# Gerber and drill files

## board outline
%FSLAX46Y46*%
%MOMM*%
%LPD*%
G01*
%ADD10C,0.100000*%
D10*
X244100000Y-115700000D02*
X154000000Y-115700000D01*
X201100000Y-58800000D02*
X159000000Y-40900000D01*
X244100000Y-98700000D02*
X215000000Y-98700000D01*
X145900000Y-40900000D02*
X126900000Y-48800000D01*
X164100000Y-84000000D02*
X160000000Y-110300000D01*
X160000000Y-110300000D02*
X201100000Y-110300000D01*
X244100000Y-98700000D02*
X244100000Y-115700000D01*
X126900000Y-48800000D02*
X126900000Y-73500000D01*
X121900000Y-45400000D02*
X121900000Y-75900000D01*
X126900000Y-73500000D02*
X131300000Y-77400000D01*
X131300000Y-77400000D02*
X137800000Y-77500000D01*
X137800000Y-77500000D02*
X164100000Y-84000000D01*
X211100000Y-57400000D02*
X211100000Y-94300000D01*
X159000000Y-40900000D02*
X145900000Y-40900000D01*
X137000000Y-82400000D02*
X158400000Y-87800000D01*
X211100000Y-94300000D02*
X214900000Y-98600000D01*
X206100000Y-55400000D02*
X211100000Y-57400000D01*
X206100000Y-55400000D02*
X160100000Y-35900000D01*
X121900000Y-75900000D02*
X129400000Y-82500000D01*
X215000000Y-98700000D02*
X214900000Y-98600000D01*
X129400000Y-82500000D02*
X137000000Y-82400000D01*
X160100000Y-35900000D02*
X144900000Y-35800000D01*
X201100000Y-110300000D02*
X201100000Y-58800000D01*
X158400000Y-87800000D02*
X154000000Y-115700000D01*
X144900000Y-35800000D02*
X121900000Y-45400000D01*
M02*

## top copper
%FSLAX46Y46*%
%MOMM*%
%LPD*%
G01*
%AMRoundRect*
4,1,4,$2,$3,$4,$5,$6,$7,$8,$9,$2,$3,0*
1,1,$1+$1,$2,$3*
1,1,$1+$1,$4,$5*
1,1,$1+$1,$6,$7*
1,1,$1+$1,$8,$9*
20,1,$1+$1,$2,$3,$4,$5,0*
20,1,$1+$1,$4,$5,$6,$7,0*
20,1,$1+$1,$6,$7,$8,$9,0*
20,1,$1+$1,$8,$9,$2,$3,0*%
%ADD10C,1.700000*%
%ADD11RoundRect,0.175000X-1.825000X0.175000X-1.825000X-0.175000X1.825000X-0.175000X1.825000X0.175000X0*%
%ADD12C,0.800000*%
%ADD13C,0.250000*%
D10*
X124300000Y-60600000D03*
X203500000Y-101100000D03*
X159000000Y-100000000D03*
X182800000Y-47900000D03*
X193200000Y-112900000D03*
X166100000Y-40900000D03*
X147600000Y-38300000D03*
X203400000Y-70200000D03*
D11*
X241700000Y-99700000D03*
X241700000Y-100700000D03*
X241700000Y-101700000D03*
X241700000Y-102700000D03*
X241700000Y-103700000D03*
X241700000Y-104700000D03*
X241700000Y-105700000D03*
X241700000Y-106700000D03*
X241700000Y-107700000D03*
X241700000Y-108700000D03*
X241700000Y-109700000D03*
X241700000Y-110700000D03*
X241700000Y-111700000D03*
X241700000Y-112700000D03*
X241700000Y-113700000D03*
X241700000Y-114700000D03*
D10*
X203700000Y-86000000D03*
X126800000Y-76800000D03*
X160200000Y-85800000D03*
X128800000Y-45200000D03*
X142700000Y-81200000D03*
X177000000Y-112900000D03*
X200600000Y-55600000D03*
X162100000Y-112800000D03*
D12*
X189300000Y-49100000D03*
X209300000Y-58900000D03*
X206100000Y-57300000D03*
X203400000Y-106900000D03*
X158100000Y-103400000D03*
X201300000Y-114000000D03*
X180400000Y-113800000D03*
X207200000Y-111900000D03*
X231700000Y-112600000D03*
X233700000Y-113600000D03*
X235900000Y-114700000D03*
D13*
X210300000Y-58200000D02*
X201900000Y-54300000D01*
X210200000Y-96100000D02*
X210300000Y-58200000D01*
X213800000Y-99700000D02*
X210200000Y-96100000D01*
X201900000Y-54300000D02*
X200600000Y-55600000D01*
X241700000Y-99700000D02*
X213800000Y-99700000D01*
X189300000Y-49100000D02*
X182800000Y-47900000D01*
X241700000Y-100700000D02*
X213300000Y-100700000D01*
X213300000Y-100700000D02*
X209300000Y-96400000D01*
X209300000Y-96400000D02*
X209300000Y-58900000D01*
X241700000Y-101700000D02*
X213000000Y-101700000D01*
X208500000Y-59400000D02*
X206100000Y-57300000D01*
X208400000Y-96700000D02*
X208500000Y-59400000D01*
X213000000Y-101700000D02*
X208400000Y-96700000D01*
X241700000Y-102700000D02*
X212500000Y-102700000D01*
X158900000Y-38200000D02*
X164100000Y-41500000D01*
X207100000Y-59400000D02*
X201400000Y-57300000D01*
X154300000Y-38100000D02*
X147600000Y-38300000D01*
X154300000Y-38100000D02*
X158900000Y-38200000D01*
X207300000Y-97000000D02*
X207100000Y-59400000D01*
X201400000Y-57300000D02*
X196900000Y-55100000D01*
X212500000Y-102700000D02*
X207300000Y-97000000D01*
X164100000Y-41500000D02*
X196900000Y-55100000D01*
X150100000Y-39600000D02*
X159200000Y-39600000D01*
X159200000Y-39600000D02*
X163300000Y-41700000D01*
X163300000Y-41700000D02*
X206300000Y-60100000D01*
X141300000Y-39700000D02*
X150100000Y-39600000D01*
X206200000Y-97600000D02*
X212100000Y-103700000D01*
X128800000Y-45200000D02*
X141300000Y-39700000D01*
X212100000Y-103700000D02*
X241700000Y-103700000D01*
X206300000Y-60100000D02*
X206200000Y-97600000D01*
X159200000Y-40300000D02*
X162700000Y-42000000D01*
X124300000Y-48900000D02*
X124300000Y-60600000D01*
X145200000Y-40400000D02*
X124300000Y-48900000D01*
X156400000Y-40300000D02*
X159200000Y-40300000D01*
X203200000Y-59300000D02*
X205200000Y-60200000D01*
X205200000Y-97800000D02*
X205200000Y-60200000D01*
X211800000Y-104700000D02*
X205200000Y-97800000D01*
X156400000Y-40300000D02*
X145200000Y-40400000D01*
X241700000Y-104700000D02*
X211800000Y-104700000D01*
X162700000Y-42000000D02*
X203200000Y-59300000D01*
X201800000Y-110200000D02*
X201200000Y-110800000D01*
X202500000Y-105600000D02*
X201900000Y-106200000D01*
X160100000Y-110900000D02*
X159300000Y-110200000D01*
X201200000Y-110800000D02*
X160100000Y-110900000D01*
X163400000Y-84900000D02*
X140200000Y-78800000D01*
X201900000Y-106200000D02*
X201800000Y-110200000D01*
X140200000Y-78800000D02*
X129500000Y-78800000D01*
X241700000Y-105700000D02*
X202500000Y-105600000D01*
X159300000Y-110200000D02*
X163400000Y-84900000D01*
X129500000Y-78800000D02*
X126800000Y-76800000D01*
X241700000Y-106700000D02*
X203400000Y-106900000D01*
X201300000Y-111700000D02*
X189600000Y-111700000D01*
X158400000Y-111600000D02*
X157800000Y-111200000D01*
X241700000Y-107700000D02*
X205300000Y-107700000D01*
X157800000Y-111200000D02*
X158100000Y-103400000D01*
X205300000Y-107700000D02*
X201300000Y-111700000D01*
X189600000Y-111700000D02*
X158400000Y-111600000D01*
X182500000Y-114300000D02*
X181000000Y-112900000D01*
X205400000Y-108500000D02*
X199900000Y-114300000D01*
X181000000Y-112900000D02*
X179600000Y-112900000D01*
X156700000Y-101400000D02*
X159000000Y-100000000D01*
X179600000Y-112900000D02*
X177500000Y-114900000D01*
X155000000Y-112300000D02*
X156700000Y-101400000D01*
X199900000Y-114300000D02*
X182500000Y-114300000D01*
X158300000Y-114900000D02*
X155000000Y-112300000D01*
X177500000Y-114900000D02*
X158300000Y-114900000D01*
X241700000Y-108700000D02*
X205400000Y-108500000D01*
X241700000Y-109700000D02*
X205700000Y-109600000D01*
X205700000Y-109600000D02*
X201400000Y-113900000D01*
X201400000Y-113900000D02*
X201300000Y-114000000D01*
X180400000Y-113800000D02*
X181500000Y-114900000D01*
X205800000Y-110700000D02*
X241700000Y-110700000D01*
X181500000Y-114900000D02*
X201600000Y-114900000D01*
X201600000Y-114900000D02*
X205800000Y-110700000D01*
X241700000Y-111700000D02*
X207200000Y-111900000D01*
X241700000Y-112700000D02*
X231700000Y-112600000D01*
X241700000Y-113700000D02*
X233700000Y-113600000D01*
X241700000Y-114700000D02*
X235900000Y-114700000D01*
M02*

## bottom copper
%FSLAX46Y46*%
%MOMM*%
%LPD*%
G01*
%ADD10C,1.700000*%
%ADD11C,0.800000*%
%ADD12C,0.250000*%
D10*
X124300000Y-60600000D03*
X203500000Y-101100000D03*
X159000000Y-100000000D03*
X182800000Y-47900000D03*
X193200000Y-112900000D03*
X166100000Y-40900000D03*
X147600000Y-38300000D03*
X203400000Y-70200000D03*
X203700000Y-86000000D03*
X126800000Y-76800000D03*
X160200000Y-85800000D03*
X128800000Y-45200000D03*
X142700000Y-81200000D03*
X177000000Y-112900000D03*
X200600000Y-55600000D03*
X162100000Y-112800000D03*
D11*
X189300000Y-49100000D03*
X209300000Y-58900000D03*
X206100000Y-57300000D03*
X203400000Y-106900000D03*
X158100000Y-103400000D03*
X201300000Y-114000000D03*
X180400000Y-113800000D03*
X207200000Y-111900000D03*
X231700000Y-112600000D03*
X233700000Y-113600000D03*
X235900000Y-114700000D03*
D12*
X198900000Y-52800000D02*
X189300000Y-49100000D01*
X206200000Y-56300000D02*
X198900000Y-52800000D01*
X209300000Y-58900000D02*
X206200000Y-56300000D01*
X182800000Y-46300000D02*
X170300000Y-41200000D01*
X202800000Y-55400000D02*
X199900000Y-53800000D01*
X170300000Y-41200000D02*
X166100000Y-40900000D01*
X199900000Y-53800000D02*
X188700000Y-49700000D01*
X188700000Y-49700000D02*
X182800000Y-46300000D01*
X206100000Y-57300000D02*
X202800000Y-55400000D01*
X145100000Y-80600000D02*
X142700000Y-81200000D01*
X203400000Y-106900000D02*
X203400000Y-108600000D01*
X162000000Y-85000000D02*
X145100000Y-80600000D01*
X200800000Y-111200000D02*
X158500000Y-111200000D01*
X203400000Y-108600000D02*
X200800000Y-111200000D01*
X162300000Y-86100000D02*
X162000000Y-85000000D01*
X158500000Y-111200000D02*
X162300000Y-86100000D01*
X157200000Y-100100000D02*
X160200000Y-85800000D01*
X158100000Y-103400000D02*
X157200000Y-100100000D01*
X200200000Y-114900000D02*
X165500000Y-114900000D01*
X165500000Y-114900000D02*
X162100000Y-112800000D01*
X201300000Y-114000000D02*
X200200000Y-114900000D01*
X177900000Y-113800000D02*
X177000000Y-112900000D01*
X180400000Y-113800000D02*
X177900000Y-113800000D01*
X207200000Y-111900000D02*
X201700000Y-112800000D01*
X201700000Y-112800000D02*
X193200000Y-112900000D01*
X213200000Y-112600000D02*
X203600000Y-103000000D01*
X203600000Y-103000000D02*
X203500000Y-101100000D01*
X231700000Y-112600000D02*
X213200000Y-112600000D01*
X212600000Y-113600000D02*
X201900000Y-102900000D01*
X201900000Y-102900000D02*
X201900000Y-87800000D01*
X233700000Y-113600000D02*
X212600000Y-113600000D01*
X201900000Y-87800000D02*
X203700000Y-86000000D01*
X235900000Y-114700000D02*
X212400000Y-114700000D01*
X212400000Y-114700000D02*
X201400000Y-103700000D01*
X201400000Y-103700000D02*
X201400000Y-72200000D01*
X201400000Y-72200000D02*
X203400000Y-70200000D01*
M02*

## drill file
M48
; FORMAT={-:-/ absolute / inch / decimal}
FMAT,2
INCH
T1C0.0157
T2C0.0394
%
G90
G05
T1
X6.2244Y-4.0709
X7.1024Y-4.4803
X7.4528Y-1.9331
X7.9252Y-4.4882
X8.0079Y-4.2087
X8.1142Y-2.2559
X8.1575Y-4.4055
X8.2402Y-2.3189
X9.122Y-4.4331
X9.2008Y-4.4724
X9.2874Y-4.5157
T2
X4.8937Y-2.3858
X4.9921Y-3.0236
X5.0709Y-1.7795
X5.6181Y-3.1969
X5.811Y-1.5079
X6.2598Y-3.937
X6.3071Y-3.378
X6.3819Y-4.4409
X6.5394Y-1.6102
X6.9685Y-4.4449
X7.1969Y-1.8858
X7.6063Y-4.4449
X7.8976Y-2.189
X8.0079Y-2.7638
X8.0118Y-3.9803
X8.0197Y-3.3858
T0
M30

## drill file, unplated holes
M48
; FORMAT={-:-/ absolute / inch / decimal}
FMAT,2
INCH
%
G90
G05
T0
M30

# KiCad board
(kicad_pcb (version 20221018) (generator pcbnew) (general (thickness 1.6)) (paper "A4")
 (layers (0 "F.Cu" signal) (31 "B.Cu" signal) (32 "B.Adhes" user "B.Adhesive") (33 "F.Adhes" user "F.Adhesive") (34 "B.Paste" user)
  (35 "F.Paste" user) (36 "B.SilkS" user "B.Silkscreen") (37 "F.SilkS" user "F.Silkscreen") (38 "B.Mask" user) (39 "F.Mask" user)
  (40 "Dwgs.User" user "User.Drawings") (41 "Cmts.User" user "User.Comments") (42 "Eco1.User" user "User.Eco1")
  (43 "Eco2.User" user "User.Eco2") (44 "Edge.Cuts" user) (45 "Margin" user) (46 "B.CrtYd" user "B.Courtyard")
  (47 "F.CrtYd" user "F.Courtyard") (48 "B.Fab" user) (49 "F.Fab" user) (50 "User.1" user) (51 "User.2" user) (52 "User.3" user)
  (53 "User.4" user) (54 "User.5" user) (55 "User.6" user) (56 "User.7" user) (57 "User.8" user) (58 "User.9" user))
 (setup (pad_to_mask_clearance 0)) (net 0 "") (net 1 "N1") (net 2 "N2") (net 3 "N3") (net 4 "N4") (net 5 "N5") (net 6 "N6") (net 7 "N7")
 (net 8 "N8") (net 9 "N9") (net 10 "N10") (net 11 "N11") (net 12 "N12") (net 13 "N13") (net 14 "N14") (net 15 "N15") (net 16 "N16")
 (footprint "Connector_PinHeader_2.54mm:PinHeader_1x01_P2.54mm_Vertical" (layer "F.Cu") (at 124.3 60.6)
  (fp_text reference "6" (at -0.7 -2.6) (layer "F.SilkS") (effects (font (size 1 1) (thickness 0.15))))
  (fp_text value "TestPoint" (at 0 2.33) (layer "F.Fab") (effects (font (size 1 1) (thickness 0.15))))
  (pad "1" thru_hole circle (at 0 0) (size 1.7 1.7) (drill 1) (layers "*.Cu" "*.Mask") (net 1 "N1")))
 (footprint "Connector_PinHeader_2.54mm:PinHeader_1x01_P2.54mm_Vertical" (layer "F.Cu") (at 203.5 101.1)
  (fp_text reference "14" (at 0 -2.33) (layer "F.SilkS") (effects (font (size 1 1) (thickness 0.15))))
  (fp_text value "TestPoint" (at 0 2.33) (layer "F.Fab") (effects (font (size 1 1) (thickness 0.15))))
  (pad "1" thru_hole circle (at 0 0) (size 1.7 1.7) (drill 1) (layers "*.Cu" "*.Mask") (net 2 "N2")))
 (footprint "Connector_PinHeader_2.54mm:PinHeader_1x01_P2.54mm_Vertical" (layer "F.Cu") (at 159 100)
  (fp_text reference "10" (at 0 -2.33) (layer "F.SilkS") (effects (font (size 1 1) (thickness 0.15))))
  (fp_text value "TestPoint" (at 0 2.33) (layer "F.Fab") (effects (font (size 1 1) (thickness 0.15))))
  (pad "1" thru_hole circle (at 0 0) (size 1.7 1.7) (drill 1) (layers "*.Cu" "*.Mask") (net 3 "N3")))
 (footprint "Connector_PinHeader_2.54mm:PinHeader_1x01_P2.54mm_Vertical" (layer "F.Cu") (at 182.8 47.9)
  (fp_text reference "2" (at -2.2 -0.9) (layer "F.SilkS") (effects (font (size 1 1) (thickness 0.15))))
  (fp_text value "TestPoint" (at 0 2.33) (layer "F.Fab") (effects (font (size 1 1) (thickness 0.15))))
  (pad "1" thru_hole circle (at 0 0) (size 1.7 1.7) (drill 1) (layers "*.Cu" "*.Mask") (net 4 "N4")))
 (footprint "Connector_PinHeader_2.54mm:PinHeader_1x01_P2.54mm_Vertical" (layer "F.Cu") (at 193.2 112.9)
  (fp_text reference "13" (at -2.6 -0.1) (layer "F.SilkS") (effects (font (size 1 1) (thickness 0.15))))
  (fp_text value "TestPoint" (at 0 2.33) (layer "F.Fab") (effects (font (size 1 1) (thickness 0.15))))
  (pad "1" thru_hole circle (at 0 0) (size 1.7 1.7) (drill 1) (layers "*.Cu" "*.Mask") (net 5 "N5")))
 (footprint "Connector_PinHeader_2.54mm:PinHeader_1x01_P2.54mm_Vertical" (layer "F.Cu") (at 166.1 40.9)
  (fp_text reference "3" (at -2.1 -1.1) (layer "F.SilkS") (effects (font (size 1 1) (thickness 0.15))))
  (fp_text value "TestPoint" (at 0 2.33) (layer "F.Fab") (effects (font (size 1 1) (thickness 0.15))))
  (pad "1" thru_hole circle (at 0 0) (size 1.7 1.7) (drill 1) (layers "*.Cu" "*.Mask") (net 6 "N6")))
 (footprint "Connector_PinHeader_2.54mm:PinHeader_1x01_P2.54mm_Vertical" (layer "F.Cu") (at 147.6 38.3)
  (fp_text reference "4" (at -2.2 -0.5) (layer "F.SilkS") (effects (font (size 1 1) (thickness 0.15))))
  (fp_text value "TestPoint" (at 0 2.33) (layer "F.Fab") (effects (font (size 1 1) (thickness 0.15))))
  (pad "1" thru_hole circle (at 0 0) (size 1.7 1.7) (drill 1) (layers "*.Cu" "*.Mask") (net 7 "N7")))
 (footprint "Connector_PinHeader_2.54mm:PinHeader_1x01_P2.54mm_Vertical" (layer "F.Cu") (at 203.4 70.2)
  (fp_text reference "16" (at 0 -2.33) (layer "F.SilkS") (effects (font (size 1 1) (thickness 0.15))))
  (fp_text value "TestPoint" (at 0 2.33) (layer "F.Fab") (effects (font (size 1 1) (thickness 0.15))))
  (pad "1" thru_hole circle (at 0 0) (size 1.7 1.7) (drill 1) (layers "*.Cu" "*.Mask") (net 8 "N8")))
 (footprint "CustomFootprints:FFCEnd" (layer "F.Cu") (at 238.7 107.2 -90)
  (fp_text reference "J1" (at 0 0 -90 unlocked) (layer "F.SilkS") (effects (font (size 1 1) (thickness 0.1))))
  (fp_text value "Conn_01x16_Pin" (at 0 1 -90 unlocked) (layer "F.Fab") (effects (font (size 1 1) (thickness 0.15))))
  (pad "1" smd roundrect (at -7.5 -3 270) (size 0.7 4) (layers "F.Cu" "F.Paste" "F.Mask") (roundrect_rratio 0.25) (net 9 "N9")
   (thermal_bridge_angle 45))
  (pad "2" smd roundrect (at -6.5 -3 270) (size 0.7 4) (layers "F.Cu" "F.Paste" "F.Mask") (roundrect_rratio 0.25) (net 4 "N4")
   (thermal_bridge_angle 45))
  (pad "3" smd roundrect (at -5.5 -3 270) (size 0.7 4) (layers "F.Cu" "F.Paste" "F.Mask") (roundrect_rratio 0.25) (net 6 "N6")
   (thermal_bridge_angle 45))
  (pad "4" smd roundrect (at -4.5 -3 270) (size 0.7 4) (layers "F.Cu" "F.Paste" "F.Mask") (roundrect_rratio 0.25) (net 7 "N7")
   (thermal_bridge_angle 45))
  (pad "5" smd roundrect (at -3.5 -3 270) (size 0.7 4) (layers "F.Cu" "F.Paste" "F.Mask") (roundrect_rratio 0.25) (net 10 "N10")
   (thermal_bridge_angle 45))
  (pad "6" smd roundrect (at -2.5 -3 270) (size 0.7 4) (layers "F.Cu" "F.Paste" "F.Mask") (roundrect_rratio 0.25) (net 1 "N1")
   (thermal_bridge_angle 45))
  (pad "7" smd roundrect (at -1.5 -3 270) (size 0.7 4) (layers "F.Cu" "F.Paste" "F.Mask") (roundrect_rratio 0.25) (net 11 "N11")
   (thermal_bridge_angle 45))
  (pad "8" smd roundrect (at -0.5 -3 270) (size 0.7 4) (layers "F.Cu" "F.Paste" "F.Mask") (roundrect_rratio 0.25) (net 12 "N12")
   (thermal_bridge_angle 45))
  (pad "9" smd roundrect (at 0.5 -3 270) (size 0.7 4) (layers "F.Cu" "F.Paste" "F.Mask") (roundrect_rratio 0.25) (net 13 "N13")
   (thermal_bridge_angle 45))
  (pad "10" smd roundrect (at 1.5 -3 270) (size 0.7 4) (layers "F.Cu" "F.Paste" "F.Mask") (roundrect_rratio 0.25) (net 3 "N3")
   (thermal_bridge_angle 45))
  (pad "11" smd roundrect (at 2.5 -3 270) (size 0.7 4) (layers "F.Cu" "F.Paste" "F.Mask") (roundrect_rratio 0.25) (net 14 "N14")
   (thermal_bridge_angle 45))
  (pad "12" smd roundrect (at 3.5 -3 270) (size 0.7 4) (layers "F.Cu" "F.Paste" "F.Mask") (roundrect_rratio 0.25) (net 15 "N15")
   (thermal_bridge_angle 45))
  (pad "13" smd roundrect (at 4.5 -3 270) (size 0.7 4) (layers "F.Cu" "F.Paste" "F.Mask") (roundrect_rratio 0.25) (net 5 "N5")
   (thermal_bridge_angle 45))
  (pad "14" smd roundrect (at 5.5 -3 270) (size 0.7 4) (layers "F.Cu" "F.Paste" "F.Mask") (roundrect_rratio 0.25) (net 2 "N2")
   (thermal_bridge_angle 45))
  (pad "15" smd roundrect (at 6.5 -3 270) (size 0.7 4) (layers "F.Cu" "F.Paste" "F.Mask") (roundrect_rratio 0.25) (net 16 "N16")
   (thermal_bridge_angle 45))
  (pad "16" smd roundrect (at 7.5 -3 270) (size 0.7 4) (layers "F.Cu" "F.Paste" "F.Mask") (roundrect_rratio 0.25) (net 8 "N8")
   (thermal_bridge_angle 45)))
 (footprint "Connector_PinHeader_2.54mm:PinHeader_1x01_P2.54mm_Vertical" (layer "F.Cu") (at 203.7 86)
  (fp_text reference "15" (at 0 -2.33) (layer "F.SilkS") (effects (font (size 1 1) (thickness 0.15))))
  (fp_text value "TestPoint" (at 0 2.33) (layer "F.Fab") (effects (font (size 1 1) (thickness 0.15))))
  (pad "1" thru_hole circle (at 0 0) (size 1.7 1.7) (drill 1) (layers "*.Cu" "*.Mask") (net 16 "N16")))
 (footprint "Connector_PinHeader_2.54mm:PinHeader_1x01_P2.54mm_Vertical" (layer "F.Cu") (at 126.8 76.8)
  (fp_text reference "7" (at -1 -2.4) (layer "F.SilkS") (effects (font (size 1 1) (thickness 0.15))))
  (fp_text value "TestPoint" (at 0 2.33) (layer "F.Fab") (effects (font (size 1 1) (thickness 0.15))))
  (pad "1" thru_hole circle (at 0 0) (size 1.7 1.7) (drill 1) (layers "*.Cu" "*.Mask") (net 11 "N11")))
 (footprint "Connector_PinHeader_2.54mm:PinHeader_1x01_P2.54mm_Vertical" (layer "F.Cu") (at 160.2 85.8)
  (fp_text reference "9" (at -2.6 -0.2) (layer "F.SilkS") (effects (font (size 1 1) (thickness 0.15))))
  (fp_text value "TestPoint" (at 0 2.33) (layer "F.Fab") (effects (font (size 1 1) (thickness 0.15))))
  (pad "1" thru_hole circle (at 0 0) (size 1.7 1.7) (drill 1) (layers "*.Cu" "*.Mask") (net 13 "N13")))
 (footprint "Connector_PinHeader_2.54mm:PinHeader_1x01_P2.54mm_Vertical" (layer "F.Cu") (at 128.8 45.2)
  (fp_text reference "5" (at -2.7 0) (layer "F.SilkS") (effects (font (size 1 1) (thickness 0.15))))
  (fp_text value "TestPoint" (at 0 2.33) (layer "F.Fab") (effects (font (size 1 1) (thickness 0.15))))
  (pad "1" thru_hole circle (at 0 0) (size 1.7 1.7) (drill 1) (layers "*.Cu" "*.Mask") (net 10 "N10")))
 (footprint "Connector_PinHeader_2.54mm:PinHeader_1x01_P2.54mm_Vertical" (layer "F.Cu") (at 142.7 81.2)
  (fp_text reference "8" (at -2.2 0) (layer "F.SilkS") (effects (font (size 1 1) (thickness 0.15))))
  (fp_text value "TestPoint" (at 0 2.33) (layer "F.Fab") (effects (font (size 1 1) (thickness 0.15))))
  (pad "1" thru_hole circle (at 0 0) (size 1.7 1.7) (drill 1) (layers "*.Cu" "*.Mask") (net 12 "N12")))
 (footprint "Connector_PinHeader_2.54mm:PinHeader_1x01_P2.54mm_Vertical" (layer "F.Cu") (at 177 112.9)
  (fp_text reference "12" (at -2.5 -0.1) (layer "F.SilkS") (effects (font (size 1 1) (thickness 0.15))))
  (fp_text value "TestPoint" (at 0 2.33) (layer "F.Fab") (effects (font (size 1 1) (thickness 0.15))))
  (pad "1" thru_hole circle (at 0 0) (size 1.7 1.7) (drill 1) (layers "*.Cu" "*.Mask") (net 15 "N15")))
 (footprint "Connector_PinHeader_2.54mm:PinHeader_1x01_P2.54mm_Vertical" (layer "F.Cu") (at 200.6 55.6)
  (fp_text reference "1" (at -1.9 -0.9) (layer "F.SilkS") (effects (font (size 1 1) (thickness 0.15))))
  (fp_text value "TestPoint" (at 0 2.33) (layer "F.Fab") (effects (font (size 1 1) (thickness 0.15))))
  (pad "1" thru_hole circle (at 0 0) (size 1.7 1.7) (drill 1) (layers "*.Cu" "*.Mask") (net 9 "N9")))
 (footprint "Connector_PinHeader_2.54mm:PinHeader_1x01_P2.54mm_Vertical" (layer "F.Cu") (at 162.1 112.8)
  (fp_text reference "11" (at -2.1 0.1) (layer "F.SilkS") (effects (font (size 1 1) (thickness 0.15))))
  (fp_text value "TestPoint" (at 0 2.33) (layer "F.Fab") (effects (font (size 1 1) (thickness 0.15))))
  (pad "1" thru_hole circle (at 0 0) (size 1.7 1.7) (drill 1) (layers "*.Cu" "*.Mask") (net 14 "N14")))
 (gr_line (start 201.1 58.8) (end 159 40.9) (stroke (width 0.1) (type default)) (layer "Edge.Cuts"))
 (gr_line (start 244.1 98.7) (end 215 98.7) (stroke (width 0.1) (type default)) (layer "Edge.Cuts"))
 (gr_line (start 244.1 115.7) (end 154 115.7) (stroke (width 0.1) (type default)) (layer "Edge.Cuts"))
 (gr_line (start 145.9 40.9) (end 126.9 48.8) (stroke (width 0.1) (type default)) (layer "Edge.Cuts"))
 (gr_line (start 164.1 84) (end 160 110.3) (stroke (width 0.1) (type default)) (layer "Edge.Cuts"))
 (gr_line (start 160 110.3) (end 201.1 110.3) (stroke (width 0.1) (type default)) (layer "Edge.Cuts"))
 (gr_line (start 244.1 98.7) (end 244.1 115.7) (stroke (width 0.1) (type default)) (layer "Edge.Cuts"))
 (gr_line (start 126.9 48.8) (end 126.9 73.5) (stroke (width 0.1) (type default)) (layer "Edge.Cuts"))
 (gr_line (start 121.9 45.4) (end 121.9 75.9) (stroke (width 0.1) (type default)) (layer "Edge.Cuts"))
 (gr_line (start 126.9 73.5) (end 131.3 77.4) (stroke (width 0.1) (type default)) (layer "Edge.Cuts"))
 (gr_line (start 131.3 77.4) (end 137.8 77.5) (stroke (width 0.1) (type default)) (layer "Edge.Cuts"))
 (gr_line (start 137.8 77.5) (end 164.1 84) (stroke (width 0.1) (type default)) (layer "Edge.Cuts"))
 (gr_line (start 211.1 57.4) (end 211.1 94.3) (stroke (width 0.1) (type default)) (layer "Edge.Cuts"))
 (gr_line (start 159 40.9) (end 145.9 40.9) (stroke (width 0.1) (type default)) (layer "Edge.Cuts"))
 (gr_line (start 137 82.4) (end 158.4 87.8) (stroke (width 0.1) (type default)) (layer "Edge.Cuts"))
 (gr_line (start 211.1 94.3) (end 214.9 98.6) (stroke (width 0.1) (type default)) (layer "Edge.Cuts"))
 (gr_line (start 206.1 55.4) (end 211.1 57.4) (stroke (width 0.1) (type default)) (layer "Edge.Cuts"))
 (gr_line (start 206.1 55.4) (end 160.1 35.9) (stroke (width 0.1) (type default)) (layer "Edge.Cuts"))
 (gr_line (start 121.9 75.9) (end 129.4 82.5) (stroke (width 0.1) (type default)) (layer "Edge.Cuts"))
 (gr_line (start 215 98.7) (end 214.9 98.6) (stroke (width 0.1) (type default)) (layer "Edge.Cuts"))
 (gr_line (start 129.4 82.5) (end 137 82.4) (stroke (width 0.1) (type default)) (layer "Edge.Cuts"))
 (gr_line (start 160.1 35.9) (end 144.9 35.8) (stroke (width 0.1) (type default)) (layer "Edge.Cuts"))
 (gr_line (start 201.1 110.3) (end 201.1 58.8) (stroke (width 0.1) (type default)) (layer "Edge.Cuts"))
 (gr_line (start 158.4 87.8) (end 154 115.7) (stroke (width 0.1) (type default)) (layer "Edge.Cuts"))
 (gr_line (start 144.9 35.8) (end 121.9 45.4) (stroke (width 0.1) (type default)) (layer "Edge.Cuts"))
 (segment (start 210.3 58.2) (end 201.9 54.3) (width 0.25) (layer "F.Cu") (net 9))
 (segment (start 210.2 96.1) (end 210.3 58.2) (width 0.25) (layer "F.Cu") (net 9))
 (segment (start 213.8 99.7) (end 210.2 96.1) (width 0.25) (layer "F.Cu") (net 9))
 (segment (start 201.9 54.3) (end 200.6 55.6) (width 0.25) (layer "F.Cu") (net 9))
 (segment (start 241.7 99.7) (end 213.8 99.7) (width 0.25) (layer "F.Cu") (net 9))
 (segment (start 189.3 49.1) (end 182.8 47.9) (width 0.25) (layer "F.Cu") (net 4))
 (segment (start 241.7 100.7) (end 213.3 100.7) (width 0.25) (layer "F.Cu") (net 4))
 (segment (start 213.3 100.7) (end 209.3 96.4) (width 0.25) (layer "F.Cu") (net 4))
 (segment (start 209.3 96.4) (end 209.3 58.9) (width 0.25) (layer "F.Cu") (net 4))
 (via (at 189.3 49.1) (size 0.8) (drill 0.4) (layers "F.Cu" "B.Cu") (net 4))
 (via (at 209.3 58.9) (size 0.8) (drill 0.4) (layers "F.Cu" "B.Cu") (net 4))
 (segment (start 198.9 52.8) (end 189.3 49.1) (width 0.25) (layer "B.Cu") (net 4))
 (segment (start 206.2 56.3) (end 198.9 52.8) (width 0.25) (layer "B.Cu") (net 4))
 (segment (start 209.3 58.9) (end 206.2 56.3) (width 0.25) (layer "B.Cu") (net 4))
 (segment (start 241.7 101.7) (end 213 101.7) (width 0.25) (layer "F.Cu") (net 6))
 (segment (start 208.5 59.4) (end 206.1 57.3) (width 0.25) (layer "F.Cu") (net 6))
 (segment (start 208.4 96.7) (end 208.5 59.4) (width 0.25) (layer "F.Cu") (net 6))
 (segment (start 213 101.7) (end 208.4 96.7) (width 0.25) (layer "F.Cu") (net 6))
 (via (at 206.1 57.3) (size 0.8) (drill 0.4) (layers "F.Cu" "B.Cu") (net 6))
 (segment (start 182.8 46.3) (end 170.3 41.2) (width 0.25) (layer "B.Cu") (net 6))
 (segment (start 202.8 55.4) (end 199.9 53.8) (width 0.25) (layer "B.Cu") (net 6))
 (segment (start 170.3 41.2) (end 166.1 40.9) (width 0.25) (layer "B.Cu") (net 6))
 (segment (start 199.9 53.8) (end 188.7 49.7) (width 0.25) (layer "B.Cu") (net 6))
 (segment (start 188.7 49.7) (end 182.8 46.3) (width 0.25) (layer "B.Cu") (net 6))
 (segment (start 206.1 57.3) (end 202.8 55.4) (width 0.25) (layer "B.Cu") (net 6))
 (segment (start 241.7 102.7) (end 212.5 102.7) (width 0.25) (layer "F.Cu") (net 7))
 (segment (start 158.9 38.2) (end 164.1 41.5) (width 0.25) (layer "F.Cu") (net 7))
 (segment (start 207.1 59.4) (end 201.4 57.3) (width 0.25) (layer "F.Cu") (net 7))
 (segment (start 154.3 38.1) (end 147.6 38.3) (width 0.25) (layer "F.Cu") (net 7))
 (segment (start 154.3 38.1) (end 158.9 38.2) (width 0.25) (layer "F.Cu") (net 7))
 (segment (start 207.3 97) (end 207.1 59.4) (width 0.25) (layer "F.Cu") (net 7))
 (segment (start 201.4 57.3) (end 196.9 55.1) (width 0.25) (layer "F.Cu") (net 7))
 (segment (start 212.5 102.7) (end 207.3 97) (width 0.25) (layer "F.Cu") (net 7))
 (segment (start 164.1 41.5) (end 196.9 55.1) (width 0.25) (layer "F.Cu") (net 7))
 (segment (start 150.1 39.6) (end 159.2 39.6) (width 0.25) (layer "F.Cu") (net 10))
 (segment (start 159.2 39.6) (end 163.3 41.7) (width 0.25) (layer "F.Cu") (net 10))
 (segment (start 163.3 41.7) (end 206.3 60.1) (width 0.25) (layer "F.Cu") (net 10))
 (segment (start 141.3 39.7) (end 150.1 39.6) (width 0.25) (layer "F.Cu") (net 10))
 (segment (start 206.2 97.6) (end 212.1 103.7) (width 0.25) (layer "F.Cu") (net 10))
 (segment (start 128.8 45.2) (end 141.3 39.7) (width 0.25) (layer "F.Cu") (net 10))
 (segment (start 212.1 103.7) (end 241.7 103.7) (width 0.25) (layer "F.Cu") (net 10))
 (segment (start 206.3 60.1) (end 206.2 97.6) (width 0.25) (layer "F.Cu") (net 10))
 (segment (start 159.2 40.3) (end 162.7 42) (width 0.25) (layer "F.Cu") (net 1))
 (segment (start 124.3 48.9) (end 124.3 60.6) (width 0.25) (layer "F.Cu") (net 1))
 (segment (start 145.2 40.4) (end 124.3 48.9) (width 0.25) (layer "F.Cu") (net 1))
 (segment (start 156.4 40.3) (end 159.2 40.3) (width 0.25) (layer "F.Cu") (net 1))
 (segment (start 203.2 59.3) (end 205.2 60.2) (width 0.25) (layer "F.Cu") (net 1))
 (segment (start 205.2 97.8) (end 205.2 60.2) (width 0.25) (layer "F.Cu") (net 1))
 (segment (start 211.8 104.7) (end 205.2 97.8) (width 0.25) (layer "F.Cu") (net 1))
 (segment (start 156.4 40.3) (end 145.2 40.4) (width 0.25) (layer "F.Cu") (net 1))
 (segment (start 241.7 104.7) (end 211.8 104.7) (width 0.25) (layer "F.Cu") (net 1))
 (segment (start 162.7 42) (end 203.2 59.3) (width 0.25) (layer "F.Cu") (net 1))
 (segment (start 201.8 110.2) (end 201.2 110.8) (width 0.25) (layer "F.Cu") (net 11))
 (segment (start 202.5 105.6) (end 201.9 106.2) (width 0.25) (layer "F.Cu") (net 11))
 (segment (start 160.1 110.9) (end 159.3 110.2) (width 0.25) (layer "F.Cu") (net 11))
 (segment (start 201.2 110.8) (end 160.1 110.9) (width 0.25) (layer "F.Cu") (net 11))
 (segment (start 163.4 84.9) (end 140.2 78.8) (width 0.25) (layer "F.Cu") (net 11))
 (segment (start 201.9 106.2) (end 201.8 110.2) (width 0.25) (layer "F.Cu") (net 11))
 (segment (start 140.2 78.8) (end 129.5 78.8) (width 0.25) (layer "F.Cu") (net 11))
 (segment (start 241.7 105.7) (end 202.5 105.6) (width 0.25) (layer "F.Cu") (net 11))
 (segment (start 159.3 110.2) (end 163.4 84.9) (width 0.25) (layer "F.Cu") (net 11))
 (segment (start 129.5 78.8) (end 126.8 76.8) (width 0.25) (layer "F.Cu") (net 11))
 (segment (start 241.7 106.7) (end 203.4 106.9) (width 0.25) (layer "F.Cu") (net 12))
 (via (at 203.4 106.9) (size 0.8) (drill 0.4) (layers "F.Cu" "B.Cu") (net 12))
 (segment (start 145.1 80.6) (end 142.7 81.2) (width 0.25) (layer "B.Cu") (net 12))
 (segment (start 203.4 106.9) (end 203.4 108.6) (width 0.25) (layer "B.Cu") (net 12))
 (segment (start 162 85) (end 145.1 80.6) (width 0.25) (layer "B.Cu") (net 12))
 (segment (start 200.8 111.2) (end 158.5 111.2) (width 0.25) (layer "B.Cu") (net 12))
 (segment (start 203.4 108.6) (end 200.8 111.2) (width 0.25) (layer "B.Cu") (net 12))
 (segment (start 162.3 86.1) (end 162 85) (width 0.25) (layer "B.Cu") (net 12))
 (segment (start 158.5 111.2) (end 162.3 86.1) (width 0.25) (layer "B.Cu") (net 12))
 (segment (start 201.3 111.7) (end 189.6 111.7) (width 0.25) (layer "F.Cu") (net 13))
 (segment (start 158.4 111.6) (end 157.8 111.2) (width 0.25) (layer "F.Cu") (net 13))
 (segment (start 241.7 107.7) (end 205.3 107.7) (width 0.25) (layer "F.Cu") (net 13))
 (segment (start 157.8 111.2) (end 158.1 103.4) (width 0.25) (layer "F.Cu") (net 13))
 (segment (start 205.3 107.7) (end 201.3 111.7) (width 0.25) (layer "F.Cu") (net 13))
 (segment (start 189.6 111.7) (end 158.4 111.6) (width 0.25) (layer "F.Cu") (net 13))
 (via (at 158.1 103.4) (size 0.8) (drill 0.4) (layers "F.Cu" "B.Cu") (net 13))
 (segment (start 157.2 100.1) (end 160.2 85.8) (width 0.25) (layer "B.Cu") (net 13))
 (segment (start 158.1 103.4) (end 157.2 100.1) (width 0.25) (layer "B.Cu") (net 13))
 (segment (start 182.5 114.3) (end 181 112.9) (width 0.25) (layer "F.Cu") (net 3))
 (segment (start 205.4 108.5) (end 199.9 114.3) (width 0.25) (layer "F.Cu") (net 3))
 (segment (start 181 112.9) (end 179.6 112.9) (width 0.25) (layer "F.Cu") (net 3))
 (segment (start 156.7 101.4) (end 159 100) (width 0.25) (layer "F.Cu") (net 3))
 (segment (start 179.6 112.9) (end 177.5 114.9) (width 0.25) (layer "F.Cu") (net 3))
 (segment (start 155 112.3) (end 156.7 101.4) (width 0.25) (layer "F.Cu") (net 3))
 (segment (start 199.9 114.3) (end 182.5 114.3) (width 0.25) (layer "F.Cu") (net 3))
 (segment (start 158.3 114.9) (end 155 112.3) (width 0.25) (layer "F.Cu") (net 3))
 (segment (start 177.5 114.9) (end 158.3 114.9) (width 0.25) (layer "F.Cu") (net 3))
 (segment (start 241.7 108.7) (end 205.4 108.5) (width 0.25) (layer "F.Cu") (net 3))
 (segment (start 241.7 109.7) (end 205.7 109.6) (width 0.25) (layer "F.Cu") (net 14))
 (segment (start 205.7 109.6) (end 201.4 113.9) (width 0.25) (layer "F.Cu") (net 14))
 (segment (start 201.4 113.9) (end 201.3 114) (width 0.25) (layer "F.Cu") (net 14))
 (via (at 201.3 114) (size 0.8) (drill 0.4) (layers "F.Cu" "B.Cu") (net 14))
 (segment (start 200.2 114.9) (end 165.5 114.9) (width 0.25) (layer "B.Cu") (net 14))
 (segment (start 165.5 114.9) (end 162.1 112.8) (width 0.25) (layer "B.Cu") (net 14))
 (segment (start 201.3 114) (end 200.2 114.9) (width 0.25) (layer "B.Cu") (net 14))
 (segment (start 180.4 113.8) (end 181.5 114.9) (width 0.25) (layer "F.Cu") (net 15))
 (segment (start 205.8 110.7) (end 241.7 110.7) (width 0.25) (layer "F.Cu") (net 15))
 (segment (start 181.5 114.9) (end 201.6 114.9) (width 0.25) (layer "F.Cu") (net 15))
 (segment (start 201.6 114.9) (end 205.8 110.7) (width 0.25) (layer "F.Cu") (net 15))
 (via (at 180.4 113.8) (size 0.8) (drill 0.4) (layers "F.Cu" "B.Cu") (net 15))
 (segment (start 177.9 113.8) (end 177 112.9) (width 0.25) (layer "B.Cu") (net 15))
 (segment (start 180.4 113.8) (end 177.9 113.8) (width 0.25) (layer "B.Cu") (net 15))
 (segment (start 241.7 111.7) (end 207.2 111.9) (width 0.25) (layer "F.Cu") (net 5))
 (via (at 207.2 111.9) (size 0.8) (drill 0.4) (layers "F.Cu" "B.Cu") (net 5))
 (segment (start 207.2 111.9) (end 201.7 112.8) (width 0.25) (layer "B.Cu") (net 5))
 (segment (start 201.7 112.8) (end 193.2 112.9) (width 0.25) (layer "B.Cu") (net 5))
 (segment (start 241.7 112.7) (end 231.7 112.6) (width 0.25) (layer "F.Cu") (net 2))
 (via (at 231.7 112.6) (size 0.8) (drill 0.4) (layers "F.Cu" "B.Cu") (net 2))
 (segment (start 213.2 112.6) (end 203.6 103) (width 0.25) (layer "B.Cu") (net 2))
 (segment (start 203.6 103) (end 203.5 101.1) (width 0.25) (layer "B.Cu") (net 2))
 (segment (start 231.7 112.6) (end 213.2 112.6) (width 0.25) (layer "B.Cu") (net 2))
 (segment (start 241.7 113.7) (end 233.7 113.6) (width 0.25) (layer "F.Cu") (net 16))
 (via (at 233.7 113.6) (size 0.8) (drill 0.4) (layers "F.Cu" "B.Cu") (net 16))
 (segment (start 212.6 113.6) (end 201.9 102.9) (width 0.25) (layer "B.Cu") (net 16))
 (segment (start 201.9 102.9) (end 201.9 87.8) (width 0.25) (layer "B.Cu") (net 16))
 (segment (start 233.7 113.6) (end 212.6 113.6) (width 0.25) (layer "B.Cu") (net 16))
 (segment (start 201.9 87.8) (end 203.7 86) (width 0.25) (layer "B.Cu") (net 16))
 (segment (start 241.7 114.7) (end 235.9 114.7) (width 0.25) (layer "F.Cu") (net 8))
 (via (at 235.9 114.7) (size 0.8) (drill 0.4) (layers "F.Cu" "B.Cu") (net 8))
 (segment (start 235.9 114.7) (end 212.4 114.7) (width 0.25) (layer "B.Cu") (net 8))
 (segment (start 212.4 114.7) (end 201.4 103.7) (width 0.25) (layer "B.Cu") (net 8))
 (segment (start 201.4 103.7) (end 201.4 72.2) (width 0.25) (layer "B.Cu") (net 8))
 (segment (start 201.4 72.2) (end 203.4 70.2) (width 0.25) (layer "B.Cu") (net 8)))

